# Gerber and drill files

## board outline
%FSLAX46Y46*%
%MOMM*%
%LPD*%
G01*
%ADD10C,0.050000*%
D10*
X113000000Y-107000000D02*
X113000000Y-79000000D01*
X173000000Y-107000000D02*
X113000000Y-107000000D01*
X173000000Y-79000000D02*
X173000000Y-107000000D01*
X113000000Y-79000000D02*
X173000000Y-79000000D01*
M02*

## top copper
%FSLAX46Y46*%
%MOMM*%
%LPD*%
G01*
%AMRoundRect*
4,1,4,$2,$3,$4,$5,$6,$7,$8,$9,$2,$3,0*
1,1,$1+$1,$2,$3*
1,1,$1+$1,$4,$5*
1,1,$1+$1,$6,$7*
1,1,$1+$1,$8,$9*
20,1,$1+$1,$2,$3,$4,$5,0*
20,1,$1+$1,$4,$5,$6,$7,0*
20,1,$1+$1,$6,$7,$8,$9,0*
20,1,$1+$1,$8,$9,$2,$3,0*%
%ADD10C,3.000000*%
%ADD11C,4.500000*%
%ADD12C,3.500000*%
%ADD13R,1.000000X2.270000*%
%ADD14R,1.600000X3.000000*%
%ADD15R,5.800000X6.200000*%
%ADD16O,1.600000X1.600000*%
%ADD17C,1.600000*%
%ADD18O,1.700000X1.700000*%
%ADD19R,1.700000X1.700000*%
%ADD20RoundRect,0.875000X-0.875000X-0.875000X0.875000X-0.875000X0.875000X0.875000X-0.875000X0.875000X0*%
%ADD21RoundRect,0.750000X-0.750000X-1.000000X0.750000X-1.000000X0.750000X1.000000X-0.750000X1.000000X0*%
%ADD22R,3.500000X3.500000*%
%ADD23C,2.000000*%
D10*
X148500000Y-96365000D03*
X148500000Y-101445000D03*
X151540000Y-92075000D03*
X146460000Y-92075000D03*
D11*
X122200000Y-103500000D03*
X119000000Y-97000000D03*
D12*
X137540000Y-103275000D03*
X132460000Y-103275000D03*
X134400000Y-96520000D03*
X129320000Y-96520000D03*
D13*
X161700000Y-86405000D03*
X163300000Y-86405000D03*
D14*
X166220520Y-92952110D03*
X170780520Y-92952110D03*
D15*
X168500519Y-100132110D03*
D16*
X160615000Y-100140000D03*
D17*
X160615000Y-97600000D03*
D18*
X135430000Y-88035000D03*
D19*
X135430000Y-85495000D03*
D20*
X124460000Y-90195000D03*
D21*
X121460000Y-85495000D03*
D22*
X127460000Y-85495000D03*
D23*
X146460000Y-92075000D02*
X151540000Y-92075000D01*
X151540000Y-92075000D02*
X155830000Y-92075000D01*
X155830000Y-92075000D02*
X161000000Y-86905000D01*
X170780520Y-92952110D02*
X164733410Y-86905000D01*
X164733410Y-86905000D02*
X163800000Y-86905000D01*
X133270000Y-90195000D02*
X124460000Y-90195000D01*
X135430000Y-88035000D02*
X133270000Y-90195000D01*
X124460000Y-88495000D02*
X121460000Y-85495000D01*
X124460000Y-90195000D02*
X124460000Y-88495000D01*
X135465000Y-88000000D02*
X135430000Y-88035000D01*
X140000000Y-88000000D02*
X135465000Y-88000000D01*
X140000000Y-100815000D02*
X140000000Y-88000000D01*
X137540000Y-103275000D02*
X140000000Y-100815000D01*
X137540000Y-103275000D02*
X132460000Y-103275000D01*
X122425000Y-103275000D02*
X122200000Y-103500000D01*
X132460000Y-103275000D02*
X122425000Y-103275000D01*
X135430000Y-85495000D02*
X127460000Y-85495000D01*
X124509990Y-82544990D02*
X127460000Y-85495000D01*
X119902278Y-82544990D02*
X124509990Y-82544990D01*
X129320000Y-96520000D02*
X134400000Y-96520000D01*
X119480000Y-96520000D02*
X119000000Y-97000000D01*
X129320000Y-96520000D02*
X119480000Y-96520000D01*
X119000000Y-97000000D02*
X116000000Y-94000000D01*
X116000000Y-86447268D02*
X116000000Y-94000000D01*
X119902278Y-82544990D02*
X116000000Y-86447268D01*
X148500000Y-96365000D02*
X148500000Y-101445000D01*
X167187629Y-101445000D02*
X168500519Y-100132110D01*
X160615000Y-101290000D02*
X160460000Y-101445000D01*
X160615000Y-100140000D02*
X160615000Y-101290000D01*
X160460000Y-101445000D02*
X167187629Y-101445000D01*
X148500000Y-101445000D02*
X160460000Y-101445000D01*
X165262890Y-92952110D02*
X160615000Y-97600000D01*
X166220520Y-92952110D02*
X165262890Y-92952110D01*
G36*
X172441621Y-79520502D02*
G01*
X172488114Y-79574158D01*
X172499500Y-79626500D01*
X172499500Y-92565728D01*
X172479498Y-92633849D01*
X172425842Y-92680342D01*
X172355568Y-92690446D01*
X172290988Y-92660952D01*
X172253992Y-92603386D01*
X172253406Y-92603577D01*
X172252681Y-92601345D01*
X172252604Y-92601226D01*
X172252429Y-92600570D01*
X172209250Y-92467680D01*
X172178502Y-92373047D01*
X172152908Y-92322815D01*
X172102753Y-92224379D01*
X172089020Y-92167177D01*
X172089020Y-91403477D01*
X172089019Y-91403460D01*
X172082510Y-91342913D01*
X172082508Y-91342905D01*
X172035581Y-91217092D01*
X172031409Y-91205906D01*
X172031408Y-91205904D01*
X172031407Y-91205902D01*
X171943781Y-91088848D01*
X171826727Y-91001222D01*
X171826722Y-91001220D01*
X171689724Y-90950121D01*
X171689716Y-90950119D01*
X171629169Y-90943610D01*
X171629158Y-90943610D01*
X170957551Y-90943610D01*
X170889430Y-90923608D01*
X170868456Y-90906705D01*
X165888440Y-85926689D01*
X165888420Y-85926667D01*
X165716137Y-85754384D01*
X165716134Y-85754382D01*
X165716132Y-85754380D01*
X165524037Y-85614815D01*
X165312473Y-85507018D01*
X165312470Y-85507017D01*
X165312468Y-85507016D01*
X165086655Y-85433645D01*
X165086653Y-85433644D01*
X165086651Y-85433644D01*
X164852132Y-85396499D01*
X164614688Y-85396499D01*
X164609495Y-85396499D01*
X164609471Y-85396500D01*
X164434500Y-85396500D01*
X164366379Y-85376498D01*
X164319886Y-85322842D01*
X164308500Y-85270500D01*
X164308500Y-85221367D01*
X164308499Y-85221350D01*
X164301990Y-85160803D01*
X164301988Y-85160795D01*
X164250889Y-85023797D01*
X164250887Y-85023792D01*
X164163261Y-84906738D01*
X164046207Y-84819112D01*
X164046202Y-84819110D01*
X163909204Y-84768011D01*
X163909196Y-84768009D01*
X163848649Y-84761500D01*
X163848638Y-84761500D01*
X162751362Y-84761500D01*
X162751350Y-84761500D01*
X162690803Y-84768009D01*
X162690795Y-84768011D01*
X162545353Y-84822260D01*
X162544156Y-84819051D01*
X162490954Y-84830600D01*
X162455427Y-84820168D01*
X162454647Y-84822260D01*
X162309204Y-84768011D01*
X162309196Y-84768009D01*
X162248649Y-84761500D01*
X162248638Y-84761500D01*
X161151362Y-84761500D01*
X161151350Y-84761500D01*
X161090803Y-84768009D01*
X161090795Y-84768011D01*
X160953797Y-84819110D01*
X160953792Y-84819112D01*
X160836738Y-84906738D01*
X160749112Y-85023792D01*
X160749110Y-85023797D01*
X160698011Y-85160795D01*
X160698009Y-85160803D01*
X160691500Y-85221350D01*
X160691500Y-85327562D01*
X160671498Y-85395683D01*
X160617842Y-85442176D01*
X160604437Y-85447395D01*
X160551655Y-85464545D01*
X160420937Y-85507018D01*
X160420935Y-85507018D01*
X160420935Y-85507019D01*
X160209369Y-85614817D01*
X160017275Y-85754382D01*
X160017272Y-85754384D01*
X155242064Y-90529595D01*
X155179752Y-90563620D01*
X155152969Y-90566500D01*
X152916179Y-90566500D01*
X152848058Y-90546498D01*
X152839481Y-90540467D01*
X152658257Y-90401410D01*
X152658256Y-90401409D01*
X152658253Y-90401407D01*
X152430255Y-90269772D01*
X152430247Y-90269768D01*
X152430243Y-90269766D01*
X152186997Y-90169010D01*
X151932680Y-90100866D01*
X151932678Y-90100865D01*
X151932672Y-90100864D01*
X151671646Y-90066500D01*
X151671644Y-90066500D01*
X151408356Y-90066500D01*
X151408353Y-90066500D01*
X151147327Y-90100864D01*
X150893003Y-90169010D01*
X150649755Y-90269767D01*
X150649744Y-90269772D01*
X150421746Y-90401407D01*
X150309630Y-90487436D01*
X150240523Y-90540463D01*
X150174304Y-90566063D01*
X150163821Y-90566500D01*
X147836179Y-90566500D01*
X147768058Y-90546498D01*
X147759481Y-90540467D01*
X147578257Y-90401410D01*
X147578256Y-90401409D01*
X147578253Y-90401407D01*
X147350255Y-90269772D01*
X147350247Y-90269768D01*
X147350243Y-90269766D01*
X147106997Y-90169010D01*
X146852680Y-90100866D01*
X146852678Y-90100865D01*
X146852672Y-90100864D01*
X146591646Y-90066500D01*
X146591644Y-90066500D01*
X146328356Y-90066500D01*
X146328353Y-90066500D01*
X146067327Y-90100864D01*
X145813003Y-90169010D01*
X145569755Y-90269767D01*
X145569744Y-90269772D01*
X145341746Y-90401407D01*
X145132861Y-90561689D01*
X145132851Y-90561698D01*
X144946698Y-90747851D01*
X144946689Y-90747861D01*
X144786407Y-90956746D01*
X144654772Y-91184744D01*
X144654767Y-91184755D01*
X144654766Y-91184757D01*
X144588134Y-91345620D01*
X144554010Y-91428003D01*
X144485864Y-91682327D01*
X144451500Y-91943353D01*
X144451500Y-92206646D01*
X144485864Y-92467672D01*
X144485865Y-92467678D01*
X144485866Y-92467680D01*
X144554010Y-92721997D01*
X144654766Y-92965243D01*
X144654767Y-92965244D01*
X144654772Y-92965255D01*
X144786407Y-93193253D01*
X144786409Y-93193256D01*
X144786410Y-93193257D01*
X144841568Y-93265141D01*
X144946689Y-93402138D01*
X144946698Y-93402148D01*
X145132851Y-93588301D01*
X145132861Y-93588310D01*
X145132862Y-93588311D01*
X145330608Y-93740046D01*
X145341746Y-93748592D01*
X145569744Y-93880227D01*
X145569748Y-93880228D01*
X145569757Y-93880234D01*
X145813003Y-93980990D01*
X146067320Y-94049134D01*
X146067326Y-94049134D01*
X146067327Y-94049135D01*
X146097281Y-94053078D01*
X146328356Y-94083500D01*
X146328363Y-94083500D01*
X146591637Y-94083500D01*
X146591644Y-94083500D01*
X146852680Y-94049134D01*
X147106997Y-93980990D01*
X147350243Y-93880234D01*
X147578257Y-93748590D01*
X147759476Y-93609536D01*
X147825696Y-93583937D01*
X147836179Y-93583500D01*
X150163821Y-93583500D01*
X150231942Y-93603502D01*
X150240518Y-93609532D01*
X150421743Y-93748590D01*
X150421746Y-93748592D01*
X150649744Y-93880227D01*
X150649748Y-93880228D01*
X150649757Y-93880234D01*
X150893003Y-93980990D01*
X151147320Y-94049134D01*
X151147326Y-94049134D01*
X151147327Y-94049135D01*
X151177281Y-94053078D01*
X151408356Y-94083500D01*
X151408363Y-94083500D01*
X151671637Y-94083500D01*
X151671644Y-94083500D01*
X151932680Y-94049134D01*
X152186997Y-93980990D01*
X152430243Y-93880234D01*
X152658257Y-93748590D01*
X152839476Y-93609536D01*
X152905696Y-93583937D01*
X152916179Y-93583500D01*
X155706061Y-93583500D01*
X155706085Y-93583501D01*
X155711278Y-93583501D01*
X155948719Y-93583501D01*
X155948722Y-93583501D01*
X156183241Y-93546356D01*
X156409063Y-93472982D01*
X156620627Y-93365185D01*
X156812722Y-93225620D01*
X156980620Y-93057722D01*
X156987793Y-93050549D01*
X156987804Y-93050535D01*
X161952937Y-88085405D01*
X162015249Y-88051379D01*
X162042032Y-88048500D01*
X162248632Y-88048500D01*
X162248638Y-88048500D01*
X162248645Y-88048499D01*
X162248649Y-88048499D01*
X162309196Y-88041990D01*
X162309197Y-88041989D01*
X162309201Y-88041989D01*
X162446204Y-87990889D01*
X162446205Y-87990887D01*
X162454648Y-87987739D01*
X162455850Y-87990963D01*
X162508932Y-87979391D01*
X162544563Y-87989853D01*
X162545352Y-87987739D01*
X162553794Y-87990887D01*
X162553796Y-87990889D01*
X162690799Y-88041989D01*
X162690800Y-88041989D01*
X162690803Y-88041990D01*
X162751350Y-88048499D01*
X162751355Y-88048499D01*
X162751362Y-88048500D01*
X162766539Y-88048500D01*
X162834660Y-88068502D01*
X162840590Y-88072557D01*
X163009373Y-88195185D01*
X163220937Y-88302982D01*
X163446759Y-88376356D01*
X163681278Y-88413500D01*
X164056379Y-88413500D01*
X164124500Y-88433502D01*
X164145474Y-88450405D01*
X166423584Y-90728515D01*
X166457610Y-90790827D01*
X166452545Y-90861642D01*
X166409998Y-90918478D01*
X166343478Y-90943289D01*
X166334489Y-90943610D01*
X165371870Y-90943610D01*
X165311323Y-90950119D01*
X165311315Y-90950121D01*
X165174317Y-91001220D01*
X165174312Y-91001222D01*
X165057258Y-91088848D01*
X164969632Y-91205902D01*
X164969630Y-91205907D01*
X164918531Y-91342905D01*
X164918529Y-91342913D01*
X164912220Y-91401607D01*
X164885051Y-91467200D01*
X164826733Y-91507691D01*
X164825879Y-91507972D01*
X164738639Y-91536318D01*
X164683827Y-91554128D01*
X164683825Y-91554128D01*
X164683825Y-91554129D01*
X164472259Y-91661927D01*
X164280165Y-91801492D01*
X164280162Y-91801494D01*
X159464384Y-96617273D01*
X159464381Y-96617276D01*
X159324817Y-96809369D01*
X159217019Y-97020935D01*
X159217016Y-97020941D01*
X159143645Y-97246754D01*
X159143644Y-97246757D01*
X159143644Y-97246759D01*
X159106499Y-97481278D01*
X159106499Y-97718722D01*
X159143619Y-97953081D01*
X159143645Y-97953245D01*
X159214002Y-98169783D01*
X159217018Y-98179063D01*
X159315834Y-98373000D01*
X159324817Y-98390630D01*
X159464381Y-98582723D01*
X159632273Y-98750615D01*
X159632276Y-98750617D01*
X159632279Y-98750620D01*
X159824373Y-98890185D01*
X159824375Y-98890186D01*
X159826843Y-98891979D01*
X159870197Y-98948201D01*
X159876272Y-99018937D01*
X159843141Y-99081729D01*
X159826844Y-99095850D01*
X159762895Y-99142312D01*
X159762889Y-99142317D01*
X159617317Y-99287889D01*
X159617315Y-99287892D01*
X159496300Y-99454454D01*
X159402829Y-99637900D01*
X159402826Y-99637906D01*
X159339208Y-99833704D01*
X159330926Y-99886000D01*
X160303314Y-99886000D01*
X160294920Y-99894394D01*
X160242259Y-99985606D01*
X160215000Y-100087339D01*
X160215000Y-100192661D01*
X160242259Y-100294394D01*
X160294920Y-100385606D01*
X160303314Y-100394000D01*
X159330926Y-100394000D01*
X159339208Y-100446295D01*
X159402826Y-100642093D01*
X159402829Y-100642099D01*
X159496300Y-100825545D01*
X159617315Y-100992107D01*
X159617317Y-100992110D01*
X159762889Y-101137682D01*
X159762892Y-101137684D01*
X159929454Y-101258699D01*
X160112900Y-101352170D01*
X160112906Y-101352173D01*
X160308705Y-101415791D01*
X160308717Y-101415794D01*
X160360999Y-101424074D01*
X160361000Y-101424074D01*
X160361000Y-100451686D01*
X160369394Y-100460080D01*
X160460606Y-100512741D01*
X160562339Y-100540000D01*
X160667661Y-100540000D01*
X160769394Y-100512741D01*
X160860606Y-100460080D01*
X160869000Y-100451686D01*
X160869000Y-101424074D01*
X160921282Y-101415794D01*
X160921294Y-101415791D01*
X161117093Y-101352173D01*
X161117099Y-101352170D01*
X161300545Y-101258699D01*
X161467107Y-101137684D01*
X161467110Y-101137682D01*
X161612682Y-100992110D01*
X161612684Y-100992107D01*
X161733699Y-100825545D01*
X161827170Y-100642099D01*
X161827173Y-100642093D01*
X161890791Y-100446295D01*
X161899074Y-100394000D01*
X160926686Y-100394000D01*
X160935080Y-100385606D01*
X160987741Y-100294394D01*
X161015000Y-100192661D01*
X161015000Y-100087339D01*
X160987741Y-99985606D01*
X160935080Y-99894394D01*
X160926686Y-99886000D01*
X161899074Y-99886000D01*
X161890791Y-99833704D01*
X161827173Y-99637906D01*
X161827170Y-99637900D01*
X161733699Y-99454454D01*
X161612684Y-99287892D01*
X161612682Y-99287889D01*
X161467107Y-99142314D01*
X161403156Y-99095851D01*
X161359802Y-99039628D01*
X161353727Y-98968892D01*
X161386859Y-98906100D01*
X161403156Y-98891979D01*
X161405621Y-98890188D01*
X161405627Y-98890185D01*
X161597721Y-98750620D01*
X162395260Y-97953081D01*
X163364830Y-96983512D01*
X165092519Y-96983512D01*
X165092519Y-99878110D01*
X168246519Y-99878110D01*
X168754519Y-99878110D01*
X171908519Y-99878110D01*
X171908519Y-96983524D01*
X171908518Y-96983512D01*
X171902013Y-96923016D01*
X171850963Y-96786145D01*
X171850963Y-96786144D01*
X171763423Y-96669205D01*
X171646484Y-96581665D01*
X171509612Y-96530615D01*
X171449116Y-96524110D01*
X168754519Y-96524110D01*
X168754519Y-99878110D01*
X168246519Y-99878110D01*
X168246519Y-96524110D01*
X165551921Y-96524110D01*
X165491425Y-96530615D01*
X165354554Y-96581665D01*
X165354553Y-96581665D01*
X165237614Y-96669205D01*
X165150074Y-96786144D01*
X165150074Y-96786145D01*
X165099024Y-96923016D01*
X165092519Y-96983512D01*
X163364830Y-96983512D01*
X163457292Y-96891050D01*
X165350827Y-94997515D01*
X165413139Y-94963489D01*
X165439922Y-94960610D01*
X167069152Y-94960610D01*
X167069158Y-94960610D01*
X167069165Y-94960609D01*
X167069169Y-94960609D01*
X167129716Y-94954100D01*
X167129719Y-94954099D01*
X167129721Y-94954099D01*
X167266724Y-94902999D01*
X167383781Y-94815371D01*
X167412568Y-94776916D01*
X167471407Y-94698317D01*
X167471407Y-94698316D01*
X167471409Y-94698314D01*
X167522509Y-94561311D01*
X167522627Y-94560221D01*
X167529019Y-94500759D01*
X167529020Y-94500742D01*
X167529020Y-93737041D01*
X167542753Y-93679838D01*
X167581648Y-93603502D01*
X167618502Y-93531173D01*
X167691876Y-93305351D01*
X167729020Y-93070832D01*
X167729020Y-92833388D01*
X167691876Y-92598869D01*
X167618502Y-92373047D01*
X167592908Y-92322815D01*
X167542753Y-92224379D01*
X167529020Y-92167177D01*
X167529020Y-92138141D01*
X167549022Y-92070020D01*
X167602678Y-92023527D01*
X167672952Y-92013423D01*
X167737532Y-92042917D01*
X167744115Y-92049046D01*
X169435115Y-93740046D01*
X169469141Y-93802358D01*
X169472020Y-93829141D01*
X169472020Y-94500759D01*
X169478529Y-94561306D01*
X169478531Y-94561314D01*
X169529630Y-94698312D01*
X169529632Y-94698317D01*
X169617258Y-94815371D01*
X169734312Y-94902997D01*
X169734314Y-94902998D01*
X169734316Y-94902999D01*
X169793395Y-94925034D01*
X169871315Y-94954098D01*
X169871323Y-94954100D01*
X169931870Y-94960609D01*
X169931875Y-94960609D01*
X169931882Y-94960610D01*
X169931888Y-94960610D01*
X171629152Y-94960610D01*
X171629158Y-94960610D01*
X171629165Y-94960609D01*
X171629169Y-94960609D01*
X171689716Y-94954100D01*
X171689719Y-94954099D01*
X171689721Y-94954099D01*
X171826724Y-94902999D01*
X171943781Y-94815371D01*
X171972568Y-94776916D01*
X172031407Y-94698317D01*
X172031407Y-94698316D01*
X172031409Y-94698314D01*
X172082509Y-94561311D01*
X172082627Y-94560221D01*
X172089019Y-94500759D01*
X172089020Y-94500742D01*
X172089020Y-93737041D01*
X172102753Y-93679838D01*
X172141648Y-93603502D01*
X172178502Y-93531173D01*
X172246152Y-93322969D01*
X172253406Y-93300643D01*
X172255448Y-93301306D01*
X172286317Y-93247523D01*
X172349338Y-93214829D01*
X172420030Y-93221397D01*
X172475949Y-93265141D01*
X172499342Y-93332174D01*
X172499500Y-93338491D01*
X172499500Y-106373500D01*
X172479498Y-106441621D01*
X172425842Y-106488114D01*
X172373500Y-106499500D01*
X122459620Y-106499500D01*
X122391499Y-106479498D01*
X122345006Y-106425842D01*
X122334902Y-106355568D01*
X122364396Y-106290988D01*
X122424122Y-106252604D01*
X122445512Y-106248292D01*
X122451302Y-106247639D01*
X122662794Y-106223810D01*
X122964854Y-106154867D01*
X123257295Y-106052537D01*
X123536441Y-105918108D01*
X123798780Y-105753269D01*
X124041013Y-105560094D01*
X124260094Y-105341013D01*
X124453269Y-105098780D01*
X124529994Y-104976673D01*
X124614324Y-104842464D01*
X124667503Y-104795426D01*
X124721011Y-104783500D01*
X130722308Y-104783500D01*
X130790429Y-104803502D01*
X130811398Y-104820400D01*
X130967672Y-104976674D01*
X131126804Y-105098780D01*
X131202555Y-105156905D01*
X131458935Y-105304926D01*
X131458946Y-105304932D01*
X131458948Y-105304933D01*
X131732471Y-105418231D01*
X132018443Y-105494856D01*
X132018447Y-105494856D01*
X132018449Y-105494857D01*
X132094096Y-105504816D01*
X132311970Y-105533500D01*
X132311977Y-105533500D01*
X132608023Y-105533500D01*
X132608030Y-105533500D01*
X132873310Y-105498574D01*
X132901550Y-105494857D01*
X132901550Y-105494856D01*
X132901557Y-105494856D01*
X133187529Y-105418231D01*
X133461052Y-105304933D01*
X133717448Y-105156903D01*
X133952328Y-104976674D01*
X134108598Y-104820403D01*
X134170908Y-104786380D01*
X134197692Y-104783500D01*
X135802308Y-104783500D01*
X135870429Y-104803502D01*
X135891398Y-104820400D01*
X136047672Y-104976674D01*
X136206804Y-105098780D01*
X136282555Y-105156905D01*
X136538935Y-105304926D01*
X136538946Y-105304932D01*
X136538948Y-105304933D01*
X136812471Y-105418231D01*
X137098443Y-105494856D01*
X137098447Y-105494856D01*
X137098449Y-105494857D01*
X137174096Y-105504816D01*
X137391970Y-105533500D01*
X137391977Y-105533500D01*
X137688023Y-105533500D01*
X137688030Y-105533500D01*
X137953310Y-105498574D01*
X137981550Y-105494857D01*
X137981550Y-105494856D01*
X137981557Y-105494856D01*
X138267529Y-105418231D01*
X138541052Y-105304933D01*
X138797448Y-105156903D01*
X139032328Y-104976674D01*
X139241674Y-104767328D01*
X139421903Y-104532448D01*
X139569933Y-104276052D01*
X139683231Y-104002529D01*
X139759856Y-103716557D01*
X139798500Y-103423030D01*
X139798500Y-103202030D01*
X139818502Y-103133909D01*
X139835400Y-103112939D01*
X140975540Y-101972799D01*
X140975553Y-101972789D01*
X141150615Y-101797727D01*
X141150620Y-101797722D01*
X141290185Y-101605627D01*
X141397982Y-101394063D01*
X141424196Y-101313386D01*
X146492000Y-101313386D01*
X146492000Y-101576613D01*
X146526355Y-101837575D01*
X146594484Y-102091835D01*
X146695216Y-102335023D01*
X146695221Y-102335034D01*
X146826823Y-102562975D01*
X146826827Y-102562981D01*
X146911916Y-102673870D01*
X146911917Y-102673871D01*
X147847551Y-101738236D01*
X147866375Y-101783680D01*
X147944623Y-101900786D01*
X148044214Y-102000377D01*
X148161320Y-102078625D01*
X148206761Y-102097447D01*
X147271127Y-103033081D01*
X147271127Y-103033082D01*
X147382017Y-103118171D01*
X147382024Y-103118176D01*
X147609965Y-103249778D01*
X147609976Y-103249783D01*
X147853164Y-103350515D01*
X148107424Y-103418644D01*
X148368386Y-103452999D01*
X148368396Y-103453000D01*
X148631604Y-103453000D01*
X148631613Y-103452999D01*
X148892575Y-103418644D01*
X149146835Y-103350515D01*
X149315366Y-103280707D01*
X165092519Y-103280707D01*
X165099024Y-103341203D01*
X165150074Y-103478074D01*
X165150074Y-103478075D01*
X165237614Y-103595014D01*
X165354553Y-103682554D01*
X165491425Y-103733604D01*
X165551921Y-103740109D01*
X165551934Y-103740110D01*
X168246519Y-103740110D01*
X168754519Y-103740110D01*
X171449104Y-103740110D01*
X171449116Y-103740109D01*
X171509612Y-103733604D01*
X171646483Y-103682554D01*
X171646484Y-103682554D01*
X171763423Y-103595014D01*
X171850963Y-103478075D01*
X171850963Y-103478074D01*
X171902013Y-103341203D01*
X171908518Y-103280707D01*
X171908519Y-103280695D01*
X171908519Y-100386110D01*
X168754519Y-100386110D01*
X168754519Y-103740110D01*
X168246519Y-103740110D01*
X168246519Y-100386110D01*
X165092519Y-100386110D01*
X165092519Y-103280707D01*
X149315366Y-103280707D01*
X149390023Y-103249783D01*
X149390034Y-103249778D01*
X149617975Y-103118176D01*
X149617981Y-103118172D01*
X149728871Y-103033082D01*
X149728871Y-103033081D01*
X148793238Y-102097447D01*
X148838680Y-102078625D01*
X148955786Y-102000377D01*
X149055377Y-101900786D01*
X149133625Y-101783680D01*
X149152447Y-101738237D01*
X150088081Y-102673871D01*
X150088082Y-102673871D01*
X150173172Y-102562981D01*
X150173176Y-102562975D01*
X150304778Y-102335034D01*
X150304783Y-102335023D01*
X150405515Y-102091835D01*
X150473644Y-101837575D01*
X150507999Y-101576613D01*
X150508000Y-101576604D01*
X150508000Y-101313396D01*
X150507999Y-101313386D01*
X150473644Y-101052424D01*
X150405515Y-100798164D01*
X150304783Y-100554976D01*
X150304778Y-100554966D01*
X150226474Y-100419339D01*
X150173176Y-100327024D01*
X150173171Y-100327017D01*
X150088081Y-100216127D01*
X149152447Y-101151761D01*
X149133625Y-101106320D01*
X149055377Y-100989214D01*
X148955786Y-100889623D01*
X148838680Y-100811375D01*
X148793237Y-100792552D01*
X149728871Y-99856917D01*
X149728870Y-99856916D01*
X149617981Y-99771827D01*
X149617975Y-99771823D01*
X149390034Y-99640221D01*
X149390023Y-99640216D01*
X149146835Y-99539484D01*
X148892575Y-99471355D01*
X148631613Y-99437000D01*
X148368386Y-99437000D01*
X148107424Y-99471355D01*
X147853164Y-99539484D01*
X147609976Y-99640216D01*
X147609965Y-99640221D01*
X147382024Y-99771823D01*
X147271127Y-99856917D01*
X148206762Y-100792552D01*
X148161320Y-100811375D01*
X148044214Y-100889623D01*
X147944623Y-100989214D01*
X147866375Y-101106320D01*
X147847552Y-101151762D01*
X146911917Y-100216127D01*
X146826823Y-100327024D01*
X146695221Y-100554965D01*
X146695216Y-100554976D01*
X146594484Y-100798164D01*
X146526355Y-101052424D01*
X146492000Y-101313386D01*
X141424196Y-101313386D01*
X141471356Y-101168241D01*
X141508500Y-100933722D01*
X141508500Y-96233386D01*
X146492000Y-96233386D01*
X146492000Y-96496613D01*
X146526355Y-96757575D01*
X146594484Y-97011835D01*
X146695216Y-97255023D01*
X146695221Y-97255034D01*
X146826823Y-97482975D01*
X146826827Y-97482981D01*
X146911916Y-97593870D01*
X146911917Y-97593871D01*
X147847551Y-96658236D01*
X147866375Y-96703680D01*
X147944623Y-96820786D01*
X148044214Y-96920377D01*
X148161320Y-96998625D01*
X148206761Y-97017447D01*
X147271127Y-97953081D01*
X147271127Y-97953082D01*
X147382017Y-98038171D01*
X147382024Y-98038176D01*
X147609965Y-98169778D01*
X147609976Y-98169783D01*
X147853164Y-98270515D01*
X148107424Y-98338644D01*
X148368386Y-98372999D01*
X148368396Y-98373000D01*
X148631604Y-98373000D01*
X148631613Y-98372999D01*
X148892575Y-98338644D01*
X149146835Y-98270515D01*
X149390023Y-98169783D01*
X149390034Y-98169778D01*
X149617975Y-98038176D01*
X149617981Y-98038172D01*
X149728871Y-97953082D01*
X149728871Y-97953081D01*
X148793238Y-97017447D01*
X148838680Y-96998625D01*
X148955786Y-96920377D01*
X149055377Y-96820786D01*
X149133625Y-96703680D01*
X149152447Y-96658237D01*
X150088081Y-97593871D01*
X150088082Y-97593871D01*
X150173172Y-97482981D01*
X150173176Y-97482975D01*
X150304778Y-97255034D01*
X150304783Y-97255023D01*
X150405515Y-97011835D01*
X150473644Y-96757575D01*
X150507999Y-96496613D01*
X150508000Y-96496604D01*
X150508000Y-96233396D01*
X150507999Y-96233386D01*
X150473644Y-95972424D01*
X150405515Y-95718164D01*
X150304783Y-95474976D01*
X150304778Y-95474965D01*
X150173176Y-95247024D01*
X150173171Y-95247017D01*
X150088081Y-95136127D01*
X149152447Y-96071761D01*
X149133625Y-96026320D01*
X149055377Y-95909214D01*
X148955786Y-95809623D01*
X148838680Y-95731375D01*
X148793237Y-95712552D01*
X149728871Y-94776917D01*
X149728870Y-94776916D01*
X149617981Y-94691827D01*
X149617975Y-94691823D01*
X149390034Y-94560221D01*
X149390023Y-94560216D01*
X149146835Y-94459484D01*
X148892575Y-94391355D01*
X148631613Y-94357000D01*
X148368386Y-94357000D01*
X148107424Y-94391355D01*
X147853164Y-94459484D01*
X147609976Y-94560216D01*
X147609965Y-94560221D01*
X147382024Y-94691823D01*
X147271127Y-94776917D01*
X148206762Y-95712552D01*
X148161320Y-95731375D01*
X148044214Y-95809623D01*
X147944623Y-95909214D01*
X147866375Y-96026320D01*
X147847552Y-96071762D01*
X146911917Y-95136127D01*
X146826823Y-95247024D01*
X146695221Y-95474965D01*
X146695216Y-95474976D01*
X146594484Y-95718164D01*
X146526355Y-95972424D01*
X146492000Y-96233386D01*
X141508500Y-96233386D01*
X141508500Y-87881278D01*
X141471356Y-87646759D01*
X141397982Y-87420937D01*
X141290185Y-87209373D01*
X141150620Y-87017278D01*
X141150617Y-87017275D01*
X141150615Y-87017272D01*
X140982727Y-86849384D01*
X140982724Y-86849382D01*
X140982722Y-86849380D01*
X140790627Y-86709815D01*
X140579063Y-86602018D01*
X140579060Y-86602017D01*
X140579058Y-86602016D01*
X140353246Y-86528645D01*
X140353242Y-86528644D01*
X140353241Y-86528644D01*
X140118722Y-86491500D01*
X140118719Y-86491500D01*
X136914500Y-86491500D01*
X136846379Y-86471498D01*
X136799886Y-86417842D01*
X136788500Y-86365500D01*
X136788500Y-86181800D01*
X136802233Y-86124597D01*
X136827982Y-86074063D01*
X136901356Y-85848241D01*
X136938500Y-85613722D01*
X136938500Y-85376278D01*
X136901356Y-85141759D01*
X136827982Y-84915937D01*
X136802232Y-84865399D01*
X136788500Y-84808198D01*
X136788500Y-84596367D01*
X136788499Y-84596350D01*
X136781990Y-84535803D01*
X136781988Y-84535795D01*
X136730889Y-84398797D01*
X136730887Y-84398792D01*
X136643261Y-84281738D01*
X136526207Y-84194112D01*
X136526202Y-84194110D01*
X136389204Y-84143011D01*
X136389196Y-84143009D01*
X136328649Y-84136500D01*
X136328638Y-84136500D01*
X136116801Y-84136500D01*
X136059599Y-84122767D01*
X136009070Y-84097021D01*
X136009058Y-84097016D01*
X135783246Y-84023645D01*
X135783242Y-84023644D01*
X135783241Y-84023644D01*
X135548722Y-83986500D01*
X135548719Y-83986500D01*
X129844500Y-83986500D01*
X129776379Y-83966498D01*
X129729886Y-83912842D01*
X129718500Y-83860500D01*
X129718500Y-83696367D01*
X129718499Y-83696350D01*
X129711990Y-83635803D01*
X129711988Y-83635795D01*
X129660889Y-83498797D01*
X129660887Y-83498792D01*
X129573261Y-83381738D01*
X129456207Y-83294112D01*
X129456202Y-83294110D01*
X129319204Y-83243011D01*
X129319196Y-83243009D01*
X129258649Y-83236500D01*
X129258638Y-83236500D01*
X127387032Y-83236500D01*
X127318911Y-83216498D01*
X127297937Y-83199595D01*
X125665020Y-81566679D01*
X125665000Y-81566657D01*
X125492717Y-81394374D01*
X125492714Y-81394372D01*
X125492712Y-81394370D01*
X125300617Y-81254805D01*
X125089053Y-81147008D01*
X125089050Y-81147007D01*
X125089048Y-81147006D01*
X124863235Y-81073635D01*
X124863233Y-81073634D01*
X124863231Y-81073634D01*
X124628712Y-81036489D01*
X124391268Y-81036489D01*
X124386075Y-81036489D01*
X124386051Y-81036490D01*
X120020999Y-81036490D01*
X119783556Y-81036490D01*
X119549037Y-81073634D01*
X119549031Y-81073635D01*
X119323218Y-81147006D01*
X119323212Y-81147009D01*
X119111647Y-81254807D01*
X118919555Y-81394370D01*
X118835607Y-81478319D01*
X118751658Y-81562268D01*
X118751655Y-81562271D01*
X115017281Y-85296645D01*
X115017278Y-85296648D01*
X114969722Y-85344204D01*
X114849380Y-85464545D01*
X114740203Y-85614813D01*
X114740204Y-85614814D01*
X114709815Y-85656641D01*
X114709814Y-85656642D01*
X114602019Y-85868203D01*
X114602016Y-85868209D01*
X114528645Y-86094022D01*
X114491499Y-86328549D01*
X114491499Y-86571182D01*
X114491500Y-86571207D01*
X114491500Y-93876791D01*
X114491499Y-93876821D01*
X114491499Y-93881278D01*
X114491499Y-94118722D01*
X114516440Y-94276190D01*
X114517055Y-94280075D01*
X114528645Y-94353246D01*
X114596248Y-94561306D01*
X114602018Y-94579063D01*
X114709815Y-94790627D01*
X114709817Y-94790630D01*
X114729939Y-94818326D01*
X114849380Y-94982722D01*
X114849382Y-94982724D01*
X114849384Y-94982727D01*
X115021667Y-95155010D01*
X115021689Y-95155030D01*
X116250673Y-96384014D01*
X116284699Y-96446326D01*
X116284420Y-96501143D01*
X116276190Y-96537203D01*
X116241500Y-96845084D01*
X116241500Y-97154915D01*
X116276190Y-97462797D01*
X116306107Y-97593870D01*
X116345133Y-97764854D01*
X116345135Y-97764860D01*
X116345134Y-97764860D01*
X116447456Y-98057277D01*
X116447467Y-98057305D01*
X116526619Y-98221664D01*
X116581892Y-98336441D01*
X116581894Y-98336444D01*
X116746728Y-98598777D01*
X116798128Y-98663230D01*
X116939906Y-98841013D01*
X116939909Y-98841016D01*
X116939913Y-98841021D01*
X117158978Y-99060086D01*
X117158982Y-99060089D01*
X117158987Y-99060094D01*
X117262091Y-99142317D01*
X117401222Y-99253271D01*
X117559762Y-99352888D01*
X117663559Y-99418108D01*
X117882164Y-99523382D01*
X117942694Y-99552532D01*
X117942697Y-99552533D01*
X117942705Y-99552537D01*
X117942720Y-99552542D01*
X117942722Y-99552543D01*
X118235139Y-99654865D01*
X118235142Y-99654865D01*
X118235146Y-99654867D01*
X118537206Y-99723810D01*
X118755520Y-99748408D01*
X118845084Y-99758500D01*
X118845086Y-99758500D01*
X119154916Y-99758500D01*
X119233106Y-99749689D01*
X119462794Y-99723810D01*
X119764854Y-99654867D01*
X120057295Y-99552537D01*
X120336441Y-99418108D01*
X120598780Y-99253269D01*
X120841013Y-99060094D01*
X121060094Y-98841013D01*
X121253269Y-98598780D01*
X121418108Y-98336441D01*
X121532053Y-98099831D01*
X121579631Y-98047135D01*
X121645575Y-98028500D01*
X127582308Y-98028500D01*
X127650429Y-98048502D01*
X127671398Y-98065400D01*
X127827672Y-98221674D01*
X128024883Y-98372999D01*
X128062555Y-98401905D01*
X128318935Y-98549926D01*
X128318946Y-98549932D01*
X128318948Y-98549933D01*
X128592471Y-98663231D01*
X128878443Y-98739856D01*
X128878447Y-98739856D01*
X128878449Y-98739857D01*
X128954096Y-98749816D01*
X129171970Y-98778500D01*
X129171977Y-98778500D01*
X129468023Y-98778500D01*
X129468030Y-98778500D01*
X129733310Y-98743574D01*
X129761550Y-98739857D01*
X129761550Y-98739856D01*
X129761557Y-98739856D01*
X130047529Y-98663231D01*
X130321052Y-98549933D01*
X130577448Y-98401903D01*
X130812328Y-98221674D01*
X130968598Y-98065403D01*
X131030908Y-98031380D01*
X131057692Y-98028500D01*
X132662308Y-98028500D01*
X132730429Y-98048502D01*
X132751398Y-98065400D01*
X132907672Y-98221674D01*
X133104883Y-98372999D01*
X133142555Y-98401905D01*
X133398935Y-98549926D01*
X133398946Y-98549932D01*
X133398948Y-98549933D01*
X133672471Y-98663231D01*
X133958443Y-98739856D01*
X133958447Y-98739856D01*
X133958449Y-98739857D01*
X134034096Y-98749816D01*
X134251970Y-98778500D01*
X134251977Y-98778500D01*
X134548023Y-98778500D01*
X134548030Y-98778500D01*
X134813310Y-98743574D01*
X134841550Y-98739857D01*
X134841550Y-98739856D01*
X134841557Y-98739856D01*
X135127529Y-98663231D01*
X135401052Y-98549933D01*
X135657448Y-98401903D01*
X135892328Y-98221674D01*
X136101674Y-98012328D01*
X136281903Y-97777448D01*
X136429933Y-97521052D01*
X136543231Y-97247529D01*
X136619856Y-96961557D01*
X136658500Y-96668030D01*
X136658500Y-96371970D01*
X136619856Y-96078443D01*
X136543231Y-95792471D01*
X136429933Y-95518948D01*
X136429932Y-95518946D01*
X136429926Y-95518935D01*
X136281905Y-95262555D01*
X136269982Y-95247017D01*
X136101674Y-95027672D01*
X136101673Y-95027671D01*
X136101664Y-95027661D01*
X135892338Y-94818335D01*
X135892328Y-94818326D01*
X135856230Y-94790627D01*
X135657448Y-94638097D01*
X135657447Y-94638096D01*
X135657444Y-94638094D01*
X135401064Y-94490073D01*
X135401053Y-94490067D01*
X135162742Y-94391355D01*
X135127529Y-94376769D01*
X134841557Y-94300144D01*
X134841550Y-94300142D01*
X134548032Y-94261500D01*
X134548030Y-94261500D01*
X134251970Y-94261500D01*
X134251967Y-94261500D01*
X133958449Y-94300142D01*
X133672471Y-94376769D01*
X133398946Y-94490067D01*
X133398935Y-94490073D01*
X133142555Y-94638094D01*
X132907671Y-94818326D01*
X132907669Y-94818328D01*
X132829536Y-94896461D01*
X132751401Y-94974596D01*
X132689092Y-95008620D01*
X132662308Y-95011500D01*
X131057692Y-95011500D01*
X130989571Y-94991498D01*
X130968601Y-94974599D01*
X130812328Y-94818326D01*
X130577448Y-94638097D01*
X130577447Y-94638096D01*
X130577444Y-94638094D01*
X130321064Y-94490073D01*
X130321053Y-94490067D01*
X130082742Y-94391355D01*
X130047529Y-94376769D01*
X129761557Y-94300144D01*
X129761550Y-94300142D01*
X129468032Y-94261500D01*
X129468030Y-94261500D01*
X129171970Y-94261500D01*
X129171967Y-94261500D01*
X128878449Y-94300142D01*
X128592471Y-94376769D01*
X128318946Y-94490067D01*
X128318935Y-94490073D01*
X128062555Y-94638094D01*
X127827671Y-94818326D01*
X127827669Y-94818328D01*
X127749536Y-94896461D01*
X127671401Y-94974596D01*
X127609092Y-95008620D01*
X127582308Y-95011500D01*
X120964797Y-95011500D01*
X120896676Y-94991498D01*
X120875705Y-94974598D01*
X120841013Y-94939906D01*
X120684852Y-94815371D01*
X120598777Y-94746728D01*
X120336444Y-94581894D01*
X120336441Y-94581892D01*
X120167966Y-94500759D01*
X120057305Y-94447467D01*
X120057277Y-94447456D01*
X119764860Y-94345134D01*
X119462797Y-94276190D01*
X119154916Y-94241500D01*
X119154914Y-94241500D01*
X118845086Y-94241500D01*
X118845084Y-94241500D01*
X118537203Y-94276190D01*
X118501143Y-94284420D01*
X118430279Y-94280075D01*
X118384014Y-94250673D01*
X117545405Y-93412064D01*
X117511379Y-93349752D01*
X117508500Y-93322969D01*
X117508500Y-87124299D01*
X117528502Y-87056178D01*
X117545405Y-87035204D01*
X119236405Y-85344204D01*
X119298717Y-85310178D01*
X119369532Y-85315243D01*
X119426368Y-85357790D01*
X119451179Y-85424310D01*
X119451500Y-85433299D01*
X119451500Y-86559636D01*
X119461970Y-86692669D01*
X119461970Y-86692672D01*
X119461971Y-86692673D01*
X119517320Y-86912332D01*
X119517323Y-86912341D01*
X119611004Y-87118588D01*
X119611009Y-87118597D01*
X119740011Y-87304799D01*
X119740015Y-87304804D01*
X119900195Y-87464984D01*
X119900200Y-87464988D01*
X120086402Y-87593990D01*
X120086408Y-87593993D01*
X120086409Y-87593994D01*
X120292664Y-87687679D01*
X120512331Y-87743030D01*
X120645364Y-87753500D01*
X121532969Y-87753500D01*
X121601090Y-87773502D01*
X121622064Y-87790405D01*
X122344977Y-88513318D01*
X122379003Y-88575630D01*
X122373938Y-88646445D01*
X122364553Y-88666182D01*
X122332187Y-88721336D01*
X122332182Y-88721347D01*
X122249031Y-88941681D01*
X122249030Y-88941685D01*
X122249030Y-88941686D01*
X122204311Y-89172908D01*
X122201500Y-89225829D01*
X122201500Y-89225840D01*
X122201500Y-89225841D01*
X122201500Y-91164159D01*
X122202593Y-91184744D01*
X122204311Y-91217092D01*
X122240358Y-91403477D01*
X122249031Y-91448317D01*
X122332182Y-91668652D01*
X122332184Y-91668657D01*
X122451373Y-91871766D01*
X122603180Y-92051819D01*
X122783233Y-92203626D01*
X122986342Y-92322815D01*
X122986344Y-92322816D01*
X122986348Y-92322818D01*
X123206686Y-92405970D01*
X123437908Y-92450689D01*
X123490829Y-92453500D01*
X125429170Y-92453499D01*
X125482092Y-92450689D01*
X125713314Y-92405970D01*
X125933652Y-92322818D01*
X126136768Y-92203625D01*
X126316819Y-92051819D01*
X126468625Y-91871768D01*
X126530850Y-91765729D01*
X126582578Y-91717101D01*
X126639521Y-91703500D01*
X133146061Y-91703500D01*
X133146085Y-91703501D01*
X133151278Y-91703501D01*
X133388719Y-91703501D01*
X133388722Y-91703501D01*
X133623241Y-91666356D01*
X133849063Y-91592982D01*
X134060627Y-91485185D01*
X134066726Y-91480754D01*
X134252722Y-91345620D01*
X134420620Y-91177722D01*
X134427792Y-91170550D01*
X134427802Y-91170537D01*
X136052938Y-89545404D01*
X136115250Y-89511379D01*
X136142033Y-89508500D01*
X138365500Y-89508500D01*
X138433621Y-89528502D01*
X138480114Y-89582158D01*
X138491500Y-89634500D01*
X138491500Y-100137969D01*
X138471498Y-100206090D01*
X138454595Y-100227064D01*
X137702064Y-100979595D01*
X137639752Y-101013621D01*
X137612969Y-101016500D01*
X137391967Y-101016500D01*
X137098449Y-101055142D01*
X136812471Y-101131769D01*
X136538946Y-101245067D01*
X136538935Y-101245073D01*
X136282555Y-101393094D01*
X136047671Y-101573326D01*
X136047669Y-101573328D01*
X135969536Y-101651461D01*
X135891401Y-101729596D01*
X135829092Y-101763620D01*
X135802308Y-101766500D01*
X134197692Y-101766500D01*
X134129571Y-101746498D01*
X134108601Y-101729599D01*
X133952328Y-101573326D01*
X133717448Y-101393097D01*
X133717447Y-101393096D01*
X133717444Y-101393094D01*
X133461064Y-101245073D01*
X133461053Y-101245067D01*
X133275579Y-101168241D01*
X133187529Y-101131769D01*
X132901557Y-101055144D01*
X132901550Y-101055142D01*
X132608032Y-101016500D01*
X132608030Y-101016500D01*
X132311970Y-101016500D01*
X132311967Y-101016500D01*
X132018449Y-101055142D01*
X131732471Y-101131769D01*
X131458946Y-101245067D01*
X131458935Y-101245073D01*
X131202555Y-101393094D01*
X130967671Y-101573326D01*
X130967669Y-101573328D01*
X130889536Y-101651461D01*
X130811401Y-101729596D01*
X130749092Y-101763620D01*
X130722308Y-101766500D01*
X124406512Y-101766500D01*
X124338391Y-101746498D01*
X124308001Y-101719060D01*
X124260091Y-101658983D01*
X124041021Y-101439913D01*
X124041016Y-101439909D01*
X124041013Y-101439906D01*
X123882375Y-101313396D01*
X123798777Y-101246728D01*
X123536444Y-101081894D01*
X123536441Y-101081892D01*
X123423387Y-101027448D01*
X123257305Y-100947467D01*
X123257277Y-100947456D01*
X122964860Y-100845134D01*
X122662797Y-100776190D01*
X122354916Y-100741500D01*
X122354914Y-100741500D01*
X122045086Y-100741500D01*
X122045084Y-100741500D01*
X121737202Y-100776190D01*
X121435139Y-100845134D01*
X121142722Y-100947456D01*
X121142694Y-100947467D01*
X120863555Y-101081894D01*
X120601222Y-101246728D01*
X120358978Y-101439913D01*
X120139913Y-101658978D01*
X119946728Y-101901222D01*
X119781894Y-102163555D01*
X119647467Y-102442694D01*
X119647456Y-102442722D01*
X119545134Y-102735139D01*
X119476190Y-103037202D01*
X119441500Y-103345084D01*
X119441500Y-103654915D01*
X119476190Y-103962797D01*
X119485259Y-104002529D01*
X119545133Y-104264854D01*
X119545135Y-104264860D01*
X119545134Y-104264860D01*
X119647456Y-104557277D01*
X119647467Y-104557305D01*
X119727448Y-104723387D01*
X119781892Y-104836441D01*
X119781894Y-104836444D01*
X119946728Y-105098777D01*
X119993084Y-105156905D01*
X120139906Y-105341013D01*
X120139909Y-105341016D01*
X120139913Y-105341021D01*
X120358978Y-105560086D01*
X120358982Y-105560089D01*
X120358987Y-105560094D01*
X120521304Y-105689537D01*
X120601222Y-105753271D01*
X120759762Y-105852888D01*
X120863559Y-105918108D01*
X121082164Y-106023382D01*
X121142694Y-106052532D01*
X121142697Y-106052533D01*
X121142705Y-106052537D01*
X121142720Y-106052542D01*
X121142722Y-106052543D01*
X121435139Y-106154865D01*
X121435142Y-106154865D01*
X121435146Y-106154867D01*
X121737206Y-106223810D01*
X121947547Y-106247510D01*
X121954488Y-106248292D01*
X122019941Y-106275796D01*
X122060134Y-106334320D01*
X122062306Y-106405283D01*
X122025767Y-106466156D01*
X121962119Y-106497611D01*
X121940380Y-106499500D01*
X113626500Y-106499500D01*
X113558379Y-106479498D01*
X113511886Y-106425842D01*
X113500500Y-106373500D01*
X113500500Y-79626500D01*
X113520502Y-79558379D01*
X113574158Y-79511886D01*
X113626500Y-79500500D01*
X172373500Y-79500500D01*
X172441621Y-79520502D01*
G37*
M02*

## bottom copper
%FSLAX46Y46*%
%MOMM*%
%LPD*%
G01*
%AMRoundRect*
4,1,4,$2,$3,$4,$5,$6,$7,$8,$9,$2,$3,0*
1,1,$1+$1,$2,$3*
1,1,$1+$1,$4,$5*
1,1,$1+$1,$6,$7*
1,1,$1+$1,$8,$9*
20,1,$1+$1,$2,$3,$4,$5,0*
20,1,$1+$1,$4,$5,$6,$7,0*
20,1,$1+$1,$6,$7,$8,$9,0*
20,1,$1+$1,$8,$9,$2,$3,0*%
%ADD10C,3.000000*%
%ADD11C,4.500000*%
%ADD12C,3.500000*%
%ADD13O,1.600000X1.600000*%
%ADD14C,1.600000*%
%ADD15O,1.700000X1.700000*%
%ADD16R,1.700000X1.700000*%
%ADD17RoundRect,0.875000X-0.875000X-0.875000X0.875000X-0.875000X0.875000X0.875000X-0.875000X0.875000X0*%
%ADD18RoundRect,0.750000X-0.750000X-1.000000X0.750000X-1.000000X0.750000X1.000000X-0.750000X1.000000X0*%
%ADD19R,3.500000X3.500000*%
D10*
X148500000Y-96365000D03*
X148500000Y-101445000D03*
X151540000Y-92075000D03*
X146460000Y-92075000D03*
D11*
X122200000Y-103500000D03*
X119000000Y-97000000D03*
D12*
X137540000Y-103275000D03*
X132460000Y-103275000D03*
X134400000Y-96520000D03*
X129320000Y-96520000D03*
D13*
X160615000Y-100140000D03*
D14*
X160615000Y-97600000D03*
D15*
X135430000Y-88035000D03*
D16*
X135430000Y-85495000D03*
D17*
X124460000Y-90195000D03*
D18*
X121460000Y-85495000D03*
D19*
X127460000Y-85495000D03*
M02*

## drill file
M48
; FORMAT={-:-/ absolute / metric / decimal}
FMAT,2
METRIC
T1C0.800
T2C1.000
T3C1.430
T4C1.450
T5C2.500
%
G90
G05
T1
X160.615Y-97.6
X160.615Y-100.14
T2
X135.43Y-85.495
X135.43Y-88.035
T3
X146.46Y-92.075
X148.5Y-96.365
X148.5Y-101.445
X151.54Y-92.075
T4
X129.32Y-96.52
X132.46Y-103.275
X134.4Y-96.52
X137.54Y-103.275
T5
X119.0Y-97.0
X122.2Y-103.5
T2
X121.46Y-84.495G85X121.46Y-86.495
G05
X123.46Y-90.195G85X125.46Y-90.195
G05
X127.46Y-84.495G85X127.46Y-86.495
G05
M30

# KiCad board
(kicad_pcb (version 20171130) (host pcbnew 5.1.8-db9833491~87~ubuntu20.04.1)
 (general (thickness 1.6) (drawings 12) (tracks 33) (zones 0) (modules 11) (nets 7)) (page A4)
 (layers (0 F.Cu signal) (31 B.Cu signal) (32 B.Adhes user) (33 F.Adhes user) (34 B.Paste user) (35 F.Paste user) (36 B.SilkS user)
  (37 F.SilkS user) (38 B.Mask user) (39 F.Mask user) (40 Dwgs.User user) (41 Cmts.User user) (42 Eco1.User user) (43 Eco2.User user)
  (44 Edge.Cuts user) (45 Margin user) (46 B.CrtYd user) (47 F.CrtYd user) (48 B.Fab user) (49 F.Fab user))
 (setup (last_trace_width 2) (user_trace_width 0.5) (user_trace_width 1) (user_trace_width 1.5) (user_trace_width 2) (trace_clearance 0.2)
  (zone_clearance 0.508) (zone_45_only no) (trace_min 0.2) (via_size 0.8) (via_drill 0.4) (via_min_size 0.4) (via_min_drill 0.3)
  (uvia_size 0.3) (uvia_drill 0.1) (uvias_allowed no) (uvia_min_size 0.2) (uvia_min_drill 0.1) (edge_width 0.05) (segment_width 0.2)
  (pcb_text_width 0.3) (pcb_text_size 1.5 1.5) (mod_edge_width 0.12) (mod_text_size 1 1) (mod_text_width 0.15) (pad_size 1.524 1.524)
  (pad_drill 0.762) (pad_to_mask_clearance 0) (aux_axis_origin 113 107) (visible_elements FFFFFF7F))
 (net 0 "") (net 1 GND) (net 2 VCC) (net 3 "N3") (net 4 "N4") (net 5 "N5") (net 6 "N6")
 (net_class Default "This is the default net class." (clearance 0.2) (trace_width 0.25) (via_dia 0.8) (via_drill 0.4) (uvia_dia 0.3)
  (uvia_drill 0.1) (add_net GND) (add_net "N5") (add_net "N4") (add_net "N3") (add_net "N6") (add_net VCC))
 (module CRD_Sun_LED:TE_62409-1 (layer F.Cu) (at 148.5 98.905 90)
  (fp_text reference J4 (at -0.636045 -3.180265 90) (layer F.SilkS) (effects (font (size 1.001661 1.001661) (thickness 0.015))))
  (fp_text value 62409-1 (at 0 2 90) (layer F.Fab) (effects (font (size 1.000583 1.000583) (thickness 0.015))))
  (pad 2 thru_hole circle (at 2.54 0 90) (size 3 3) (drill 1.43) (layers *.Cu *.Mask) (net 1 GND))
  (pad 1 thru_hole circle (at -2.54 0 90) (size 3 3) (drill 1.43) (layers *.Cu *.Mask) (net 1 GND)))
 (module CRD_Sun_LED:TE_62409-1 (layer F.Cu) (at 149 92.075)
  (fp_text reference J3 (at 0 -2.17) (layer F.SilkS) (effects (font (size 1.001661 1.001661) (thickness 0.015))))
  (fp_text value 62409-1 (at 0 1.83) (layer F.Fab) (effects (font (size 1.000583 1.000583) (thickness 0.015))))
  (pad 2 thru_hole circle (at 2.54 0) (size 3 3) (drill 1.43) (layers *.Cu *.Mask) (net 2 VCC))
  (pad 1 thru_hole circle (at -2.54 0) (size 3 3) (drill 1.43) (layers *.Cu *.Mask) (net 2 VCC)))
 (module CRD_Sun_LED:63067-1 (layer F.Cu) (at 118 103)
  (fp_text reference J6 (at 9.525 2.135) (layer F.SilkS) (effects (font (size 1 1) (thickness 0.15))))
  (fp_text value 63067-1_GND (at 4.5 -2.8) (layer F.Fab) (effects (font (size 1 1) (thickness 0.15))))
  (pad 1 thru_hole circle (at 4.2 0.5) (size 4.5 4.5) (drill 2.5) (layers *.Cu *.Mask) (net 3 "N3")))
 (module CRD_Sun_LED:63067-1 (layer F.Cu) (at 114.8 96.5)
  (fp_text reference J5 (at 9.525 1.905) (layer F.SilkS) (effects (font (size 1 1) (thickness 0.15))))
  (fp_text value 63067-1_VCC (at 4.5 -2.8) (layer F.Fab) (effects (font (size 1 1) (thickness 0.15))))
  (pad 1 thru_hole circle (at 4.2 0.5) (size 4.5 4.5) (drill 2.5) (layers *.Cu *.Mask) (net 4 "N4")))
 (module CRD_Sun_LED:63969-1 (layer F.Cu) (at 135 103.275)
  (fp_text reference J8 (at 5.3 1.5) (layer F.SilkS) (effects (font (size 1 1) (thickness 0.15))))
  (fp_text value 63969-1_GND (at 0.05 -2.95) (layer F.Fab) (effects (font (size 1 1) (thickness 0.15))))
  (pad 1 thru_hole circle (at 2.54 0) (size 3.5 3.5) (drill 1.45) (layers *.Cu *.Mask) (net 3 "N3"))
  (pad 1 thru_hole circle (at -2.54 0) (size 3.5 3.5) (drill 1.45) (layers *.Cu *.Mask) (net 3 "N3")))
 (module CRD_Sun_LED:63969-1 (layer F.Cu) (at 131.86 96.52)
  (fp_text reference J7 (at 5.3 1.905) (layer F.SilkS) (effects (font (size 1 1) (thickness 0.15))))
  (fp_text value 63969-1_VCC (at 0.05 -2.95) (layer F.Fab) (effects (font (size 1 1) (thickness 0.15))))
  (pad 1 thru_hole circle (at 2.54 0) (size 3.5 3.5) (drill 1.45) (layers *.Cu *.Mask) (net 4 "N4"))
  (pad 1 thru_hole circle (at -2.54 0) (size 3.5 3.5) (drill 1.45) (layers *.Cu *.Mask) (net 4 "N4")))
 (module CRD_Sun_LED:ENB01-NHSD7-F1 (layer F.Cu) (at 164 84.905 270)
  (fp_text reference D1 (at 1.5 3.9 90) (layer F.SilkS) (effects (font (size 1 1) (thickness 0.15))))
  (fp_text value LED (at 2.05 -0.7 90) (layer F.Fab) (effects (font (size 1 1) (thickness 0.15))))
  (pad 2 smd rect (at 1.5 2.3 270) (size 2.27 1) (layers F.Cu F.Paste F.Mask) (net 2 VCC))
  (pad 1 smd rect (at 1.5 0.7 270) (size 2.27 1) (layers F.Cu F.Paste F.Mask) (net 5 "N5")))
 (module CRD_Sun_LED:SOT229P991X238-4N (layer F.Cu) (at 168.5 97.405 270)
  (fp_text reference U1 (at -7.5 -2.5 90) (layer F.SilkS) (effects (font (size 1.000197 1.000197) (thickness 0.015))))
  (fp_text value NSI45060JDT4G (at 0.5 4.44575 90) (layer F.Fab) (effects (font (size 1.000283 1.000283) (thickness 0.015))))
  (pad 3 smd rect (at -4.45289 2.27948 270) (size 3 1.6) (layers F.Cu F.Paste F.Mask) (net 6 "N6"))
  (pad 1 smd rect (at -4.45289 -2.28052 270) (size 3 1.6) (layers F.Cu F.Paste F.Mask) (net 5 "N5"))
  (pad 4 smd rect (at 2.72711 -0.000519 270) (size 6.2 5.8) (layers F.Cu F.Paste F.Mask) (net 1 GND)))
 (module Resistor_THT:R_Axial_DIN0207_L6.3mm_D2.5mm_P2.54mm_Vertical (layer F.Cu) (at 160.615 97.6 270)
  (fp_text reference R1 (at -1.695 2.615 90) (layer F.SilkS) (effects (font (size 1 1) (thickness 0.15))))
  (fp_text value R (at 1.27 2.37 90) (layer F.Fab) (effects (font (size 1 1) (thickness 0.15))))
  (pad 2 thru_hole oval (at 2.54 0 270) (size 1.6 1.6) (drill 0.8) (layers *.Cu *.Mask) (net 1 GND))
  (pad 1 thru_hole circle (at 0 0 270) (size 1.6 1.6) (drill 0.8) (layers *.Cu *.Mask) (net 6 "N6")))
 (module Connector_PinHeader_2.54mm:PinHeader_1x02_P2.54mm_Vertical (layer F.Cu) (at 135.43 85.495)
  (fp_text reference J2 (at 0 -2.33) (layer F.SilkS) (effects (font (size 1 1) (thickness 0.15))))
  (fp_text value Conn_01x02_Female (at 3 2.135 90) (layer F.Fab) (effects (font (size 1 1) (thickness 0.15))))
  (pad 2 thru_hole oval (at 0 2.54) (size 1.7 1.7) (drill 1) (layers *.Cu *.Mask) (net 3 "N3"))
  (pad 1 thru_hole rect (at 0 0) (size 1.7 1.7) (drill 1) (layers *.Cu *.Mask) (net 4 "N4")))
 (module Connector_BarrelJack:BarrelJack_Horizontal (layer F.Cu) (at 127.46 85.495)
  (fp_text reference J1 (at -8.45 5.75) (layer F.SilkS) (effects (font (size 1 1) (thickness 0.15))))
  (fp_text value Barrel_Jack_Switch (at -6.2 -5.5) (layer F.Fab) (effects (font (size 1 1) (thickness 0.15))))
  (pad 3 thru_hole roundrect (at -3 4.7) (size 3.5 3.5) (drill oval 3 1) (layers *.Cu *.Mask) (roundrect_rratio 0.25) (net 3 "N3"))
  (pad 2 thru_hole roundrect (at -6 0) (size 3 3.5) (drill oval 1 3) (layers *.Cu *.Mask) (roundrect_rratio 0.25) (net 3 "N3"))
  (pad 1 thru_hole rect (at 0 0) (size 3.5 3.5) (drill oval 1 3) (layers *.Cu *.Mask) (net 4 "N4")))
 (gr_line (start 113 107) (end 113 79) (layer Edge.Cuts) (width 0.05))
 (gr_line (start 173 107) (end 113 107) (layer Edge.Cuts) (width 0.05))
 (gr_line (start 173 79) (end 173 107) (layer Edge.Cuts) (width 0.05))
 (gr_line (start 113 79) (end 173 79) (layer Edge.Cuts) (width 0.05))
 (segment (start 146.46 92.075) (end 151.54 92.075) (width 2) (layer F.Cu) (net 2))
 (segment (start 151.54 92.075) (end 155.83 92.075) (width 2) (layer F.Cu) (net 2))
 (segment (start 155.83 92.075) (end 161 86.905) (width 2) (layer F.Cu) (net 2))
 (segment (start 170.78052 92.95211) (end 164.73341 86.905) (width 2) (layer F.Cu) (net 5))
 (segment (start 164.73341 86.905) (end 163.8 86.905) (width 2) (layer F.Cu) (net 5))
 (segment (start 133.27 90.195) (end 124.46 90.195) (width 2) (layer F.Cu) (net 3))
 (segment (start 135.43 88.035) (end 133.27 90.195) (width 2) (layer F.Cu) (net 3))
 (segment (start 124.46 88.495) (end 121.46 85.495) (width 2) (layer F.Cu) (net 3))
 (segment (start 124.46 90.195) (end 124.46 88.495) (width 2) (layer F.Cu) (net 3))
 (segment (start 135.465 88) (end 135.43 88.035) (width 2) (layer F.Cu) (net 3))
 (segment (start 140 88) (end 135.465 88) (width 2) (layer F.Cu) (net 3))
 (segment (start 140 100.815) (end 140 88) (width 2) (layer F.Cu) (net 3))
 (segment (start 137.54 103.275) (end 140 100.815) (width 2) (layer F.Cu) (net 3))
 (segment (start 137.54 103.275) (end 132.46 103.275) (width 2) (layer F.Cu) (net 3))
 (segment (start 122.425 103.275) (end 122.2 103.5) (width 2) (layer F.Cu) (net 3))
 (segment (start 132.46 103.275) (end 122.425 103.275) (width 2) (layer F.Cu) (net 3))
 (segment (start 135.43 85.495) (end 127.46 85.495) (width 2) (layer F.Cu) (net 4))
 (segment (start 124.50999 82.54499) (end 127.46 85.495) (width 2) (layer F.Cu) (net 4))
 (segment (start 119.902278 82.54499) (end 124.50999 82.54499) (width 2) (layer F.Cu) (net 4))
 (segment (start 129.32 96.52) (end 134.4 96.52) (width 2) (layer F.Cu) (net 4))
 (segment (start 119.48 96.52) (end 119 97) (width 2) (layer F.Cu) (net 4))
 (segment (start 129.32 96.52) (end 119.48 96.52) (width 2) (layer F.Cu) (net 4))
 (segment (start 119 97) (end 116 94) (width 2) (layer F.Cu) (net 4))
 (segment (start 116 86.447268) (end 116 94) (width 2) (layer F.Cu) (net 4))
 (segment (start 119.902278 82.54499) (end 116 86.447268) (width 2) (layer F.Cu) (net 4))
 (segment (start 148.5 96.365) (end 148.5 101.445) (width 2) (layer F.Cu) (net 1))
 (segment (start 167.187629 101.445) (end 168.500519 100.13211) (width 2) (layer F.Cu) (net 1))
 (segment (start 160.615 101.29) (end 160.46 101.445) (width 2) (layer F.Cu) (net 1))
 (segment (start 160.615 100.14) (end 160.615 101.29) (width 2) (layer F.Cu) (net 1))
 (segment (start 160.46 101.445) (end 167.187629 101.445) (width 2) (layer F.Cu) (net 1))
 (segment (start 148.5 101.445) (end 160.46 101.445) (width 2) (layer F.Cu) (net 1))
 (segment (start 165.26289 92.95211) (end 160.615 97.6) (width 2) (layer F.Cu) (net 6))
 (segment (start 166.22052 92.95211) (end 165.26289 92.95211) (width 2) (layer F.Cu) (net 6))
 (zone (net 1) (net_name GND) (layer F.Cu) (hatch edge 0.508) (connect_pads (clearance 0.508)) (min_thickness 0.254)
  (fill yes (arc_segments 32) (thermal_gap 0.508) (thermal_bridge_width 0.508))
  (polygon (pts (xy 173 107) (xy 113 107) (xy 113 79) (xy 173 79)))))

